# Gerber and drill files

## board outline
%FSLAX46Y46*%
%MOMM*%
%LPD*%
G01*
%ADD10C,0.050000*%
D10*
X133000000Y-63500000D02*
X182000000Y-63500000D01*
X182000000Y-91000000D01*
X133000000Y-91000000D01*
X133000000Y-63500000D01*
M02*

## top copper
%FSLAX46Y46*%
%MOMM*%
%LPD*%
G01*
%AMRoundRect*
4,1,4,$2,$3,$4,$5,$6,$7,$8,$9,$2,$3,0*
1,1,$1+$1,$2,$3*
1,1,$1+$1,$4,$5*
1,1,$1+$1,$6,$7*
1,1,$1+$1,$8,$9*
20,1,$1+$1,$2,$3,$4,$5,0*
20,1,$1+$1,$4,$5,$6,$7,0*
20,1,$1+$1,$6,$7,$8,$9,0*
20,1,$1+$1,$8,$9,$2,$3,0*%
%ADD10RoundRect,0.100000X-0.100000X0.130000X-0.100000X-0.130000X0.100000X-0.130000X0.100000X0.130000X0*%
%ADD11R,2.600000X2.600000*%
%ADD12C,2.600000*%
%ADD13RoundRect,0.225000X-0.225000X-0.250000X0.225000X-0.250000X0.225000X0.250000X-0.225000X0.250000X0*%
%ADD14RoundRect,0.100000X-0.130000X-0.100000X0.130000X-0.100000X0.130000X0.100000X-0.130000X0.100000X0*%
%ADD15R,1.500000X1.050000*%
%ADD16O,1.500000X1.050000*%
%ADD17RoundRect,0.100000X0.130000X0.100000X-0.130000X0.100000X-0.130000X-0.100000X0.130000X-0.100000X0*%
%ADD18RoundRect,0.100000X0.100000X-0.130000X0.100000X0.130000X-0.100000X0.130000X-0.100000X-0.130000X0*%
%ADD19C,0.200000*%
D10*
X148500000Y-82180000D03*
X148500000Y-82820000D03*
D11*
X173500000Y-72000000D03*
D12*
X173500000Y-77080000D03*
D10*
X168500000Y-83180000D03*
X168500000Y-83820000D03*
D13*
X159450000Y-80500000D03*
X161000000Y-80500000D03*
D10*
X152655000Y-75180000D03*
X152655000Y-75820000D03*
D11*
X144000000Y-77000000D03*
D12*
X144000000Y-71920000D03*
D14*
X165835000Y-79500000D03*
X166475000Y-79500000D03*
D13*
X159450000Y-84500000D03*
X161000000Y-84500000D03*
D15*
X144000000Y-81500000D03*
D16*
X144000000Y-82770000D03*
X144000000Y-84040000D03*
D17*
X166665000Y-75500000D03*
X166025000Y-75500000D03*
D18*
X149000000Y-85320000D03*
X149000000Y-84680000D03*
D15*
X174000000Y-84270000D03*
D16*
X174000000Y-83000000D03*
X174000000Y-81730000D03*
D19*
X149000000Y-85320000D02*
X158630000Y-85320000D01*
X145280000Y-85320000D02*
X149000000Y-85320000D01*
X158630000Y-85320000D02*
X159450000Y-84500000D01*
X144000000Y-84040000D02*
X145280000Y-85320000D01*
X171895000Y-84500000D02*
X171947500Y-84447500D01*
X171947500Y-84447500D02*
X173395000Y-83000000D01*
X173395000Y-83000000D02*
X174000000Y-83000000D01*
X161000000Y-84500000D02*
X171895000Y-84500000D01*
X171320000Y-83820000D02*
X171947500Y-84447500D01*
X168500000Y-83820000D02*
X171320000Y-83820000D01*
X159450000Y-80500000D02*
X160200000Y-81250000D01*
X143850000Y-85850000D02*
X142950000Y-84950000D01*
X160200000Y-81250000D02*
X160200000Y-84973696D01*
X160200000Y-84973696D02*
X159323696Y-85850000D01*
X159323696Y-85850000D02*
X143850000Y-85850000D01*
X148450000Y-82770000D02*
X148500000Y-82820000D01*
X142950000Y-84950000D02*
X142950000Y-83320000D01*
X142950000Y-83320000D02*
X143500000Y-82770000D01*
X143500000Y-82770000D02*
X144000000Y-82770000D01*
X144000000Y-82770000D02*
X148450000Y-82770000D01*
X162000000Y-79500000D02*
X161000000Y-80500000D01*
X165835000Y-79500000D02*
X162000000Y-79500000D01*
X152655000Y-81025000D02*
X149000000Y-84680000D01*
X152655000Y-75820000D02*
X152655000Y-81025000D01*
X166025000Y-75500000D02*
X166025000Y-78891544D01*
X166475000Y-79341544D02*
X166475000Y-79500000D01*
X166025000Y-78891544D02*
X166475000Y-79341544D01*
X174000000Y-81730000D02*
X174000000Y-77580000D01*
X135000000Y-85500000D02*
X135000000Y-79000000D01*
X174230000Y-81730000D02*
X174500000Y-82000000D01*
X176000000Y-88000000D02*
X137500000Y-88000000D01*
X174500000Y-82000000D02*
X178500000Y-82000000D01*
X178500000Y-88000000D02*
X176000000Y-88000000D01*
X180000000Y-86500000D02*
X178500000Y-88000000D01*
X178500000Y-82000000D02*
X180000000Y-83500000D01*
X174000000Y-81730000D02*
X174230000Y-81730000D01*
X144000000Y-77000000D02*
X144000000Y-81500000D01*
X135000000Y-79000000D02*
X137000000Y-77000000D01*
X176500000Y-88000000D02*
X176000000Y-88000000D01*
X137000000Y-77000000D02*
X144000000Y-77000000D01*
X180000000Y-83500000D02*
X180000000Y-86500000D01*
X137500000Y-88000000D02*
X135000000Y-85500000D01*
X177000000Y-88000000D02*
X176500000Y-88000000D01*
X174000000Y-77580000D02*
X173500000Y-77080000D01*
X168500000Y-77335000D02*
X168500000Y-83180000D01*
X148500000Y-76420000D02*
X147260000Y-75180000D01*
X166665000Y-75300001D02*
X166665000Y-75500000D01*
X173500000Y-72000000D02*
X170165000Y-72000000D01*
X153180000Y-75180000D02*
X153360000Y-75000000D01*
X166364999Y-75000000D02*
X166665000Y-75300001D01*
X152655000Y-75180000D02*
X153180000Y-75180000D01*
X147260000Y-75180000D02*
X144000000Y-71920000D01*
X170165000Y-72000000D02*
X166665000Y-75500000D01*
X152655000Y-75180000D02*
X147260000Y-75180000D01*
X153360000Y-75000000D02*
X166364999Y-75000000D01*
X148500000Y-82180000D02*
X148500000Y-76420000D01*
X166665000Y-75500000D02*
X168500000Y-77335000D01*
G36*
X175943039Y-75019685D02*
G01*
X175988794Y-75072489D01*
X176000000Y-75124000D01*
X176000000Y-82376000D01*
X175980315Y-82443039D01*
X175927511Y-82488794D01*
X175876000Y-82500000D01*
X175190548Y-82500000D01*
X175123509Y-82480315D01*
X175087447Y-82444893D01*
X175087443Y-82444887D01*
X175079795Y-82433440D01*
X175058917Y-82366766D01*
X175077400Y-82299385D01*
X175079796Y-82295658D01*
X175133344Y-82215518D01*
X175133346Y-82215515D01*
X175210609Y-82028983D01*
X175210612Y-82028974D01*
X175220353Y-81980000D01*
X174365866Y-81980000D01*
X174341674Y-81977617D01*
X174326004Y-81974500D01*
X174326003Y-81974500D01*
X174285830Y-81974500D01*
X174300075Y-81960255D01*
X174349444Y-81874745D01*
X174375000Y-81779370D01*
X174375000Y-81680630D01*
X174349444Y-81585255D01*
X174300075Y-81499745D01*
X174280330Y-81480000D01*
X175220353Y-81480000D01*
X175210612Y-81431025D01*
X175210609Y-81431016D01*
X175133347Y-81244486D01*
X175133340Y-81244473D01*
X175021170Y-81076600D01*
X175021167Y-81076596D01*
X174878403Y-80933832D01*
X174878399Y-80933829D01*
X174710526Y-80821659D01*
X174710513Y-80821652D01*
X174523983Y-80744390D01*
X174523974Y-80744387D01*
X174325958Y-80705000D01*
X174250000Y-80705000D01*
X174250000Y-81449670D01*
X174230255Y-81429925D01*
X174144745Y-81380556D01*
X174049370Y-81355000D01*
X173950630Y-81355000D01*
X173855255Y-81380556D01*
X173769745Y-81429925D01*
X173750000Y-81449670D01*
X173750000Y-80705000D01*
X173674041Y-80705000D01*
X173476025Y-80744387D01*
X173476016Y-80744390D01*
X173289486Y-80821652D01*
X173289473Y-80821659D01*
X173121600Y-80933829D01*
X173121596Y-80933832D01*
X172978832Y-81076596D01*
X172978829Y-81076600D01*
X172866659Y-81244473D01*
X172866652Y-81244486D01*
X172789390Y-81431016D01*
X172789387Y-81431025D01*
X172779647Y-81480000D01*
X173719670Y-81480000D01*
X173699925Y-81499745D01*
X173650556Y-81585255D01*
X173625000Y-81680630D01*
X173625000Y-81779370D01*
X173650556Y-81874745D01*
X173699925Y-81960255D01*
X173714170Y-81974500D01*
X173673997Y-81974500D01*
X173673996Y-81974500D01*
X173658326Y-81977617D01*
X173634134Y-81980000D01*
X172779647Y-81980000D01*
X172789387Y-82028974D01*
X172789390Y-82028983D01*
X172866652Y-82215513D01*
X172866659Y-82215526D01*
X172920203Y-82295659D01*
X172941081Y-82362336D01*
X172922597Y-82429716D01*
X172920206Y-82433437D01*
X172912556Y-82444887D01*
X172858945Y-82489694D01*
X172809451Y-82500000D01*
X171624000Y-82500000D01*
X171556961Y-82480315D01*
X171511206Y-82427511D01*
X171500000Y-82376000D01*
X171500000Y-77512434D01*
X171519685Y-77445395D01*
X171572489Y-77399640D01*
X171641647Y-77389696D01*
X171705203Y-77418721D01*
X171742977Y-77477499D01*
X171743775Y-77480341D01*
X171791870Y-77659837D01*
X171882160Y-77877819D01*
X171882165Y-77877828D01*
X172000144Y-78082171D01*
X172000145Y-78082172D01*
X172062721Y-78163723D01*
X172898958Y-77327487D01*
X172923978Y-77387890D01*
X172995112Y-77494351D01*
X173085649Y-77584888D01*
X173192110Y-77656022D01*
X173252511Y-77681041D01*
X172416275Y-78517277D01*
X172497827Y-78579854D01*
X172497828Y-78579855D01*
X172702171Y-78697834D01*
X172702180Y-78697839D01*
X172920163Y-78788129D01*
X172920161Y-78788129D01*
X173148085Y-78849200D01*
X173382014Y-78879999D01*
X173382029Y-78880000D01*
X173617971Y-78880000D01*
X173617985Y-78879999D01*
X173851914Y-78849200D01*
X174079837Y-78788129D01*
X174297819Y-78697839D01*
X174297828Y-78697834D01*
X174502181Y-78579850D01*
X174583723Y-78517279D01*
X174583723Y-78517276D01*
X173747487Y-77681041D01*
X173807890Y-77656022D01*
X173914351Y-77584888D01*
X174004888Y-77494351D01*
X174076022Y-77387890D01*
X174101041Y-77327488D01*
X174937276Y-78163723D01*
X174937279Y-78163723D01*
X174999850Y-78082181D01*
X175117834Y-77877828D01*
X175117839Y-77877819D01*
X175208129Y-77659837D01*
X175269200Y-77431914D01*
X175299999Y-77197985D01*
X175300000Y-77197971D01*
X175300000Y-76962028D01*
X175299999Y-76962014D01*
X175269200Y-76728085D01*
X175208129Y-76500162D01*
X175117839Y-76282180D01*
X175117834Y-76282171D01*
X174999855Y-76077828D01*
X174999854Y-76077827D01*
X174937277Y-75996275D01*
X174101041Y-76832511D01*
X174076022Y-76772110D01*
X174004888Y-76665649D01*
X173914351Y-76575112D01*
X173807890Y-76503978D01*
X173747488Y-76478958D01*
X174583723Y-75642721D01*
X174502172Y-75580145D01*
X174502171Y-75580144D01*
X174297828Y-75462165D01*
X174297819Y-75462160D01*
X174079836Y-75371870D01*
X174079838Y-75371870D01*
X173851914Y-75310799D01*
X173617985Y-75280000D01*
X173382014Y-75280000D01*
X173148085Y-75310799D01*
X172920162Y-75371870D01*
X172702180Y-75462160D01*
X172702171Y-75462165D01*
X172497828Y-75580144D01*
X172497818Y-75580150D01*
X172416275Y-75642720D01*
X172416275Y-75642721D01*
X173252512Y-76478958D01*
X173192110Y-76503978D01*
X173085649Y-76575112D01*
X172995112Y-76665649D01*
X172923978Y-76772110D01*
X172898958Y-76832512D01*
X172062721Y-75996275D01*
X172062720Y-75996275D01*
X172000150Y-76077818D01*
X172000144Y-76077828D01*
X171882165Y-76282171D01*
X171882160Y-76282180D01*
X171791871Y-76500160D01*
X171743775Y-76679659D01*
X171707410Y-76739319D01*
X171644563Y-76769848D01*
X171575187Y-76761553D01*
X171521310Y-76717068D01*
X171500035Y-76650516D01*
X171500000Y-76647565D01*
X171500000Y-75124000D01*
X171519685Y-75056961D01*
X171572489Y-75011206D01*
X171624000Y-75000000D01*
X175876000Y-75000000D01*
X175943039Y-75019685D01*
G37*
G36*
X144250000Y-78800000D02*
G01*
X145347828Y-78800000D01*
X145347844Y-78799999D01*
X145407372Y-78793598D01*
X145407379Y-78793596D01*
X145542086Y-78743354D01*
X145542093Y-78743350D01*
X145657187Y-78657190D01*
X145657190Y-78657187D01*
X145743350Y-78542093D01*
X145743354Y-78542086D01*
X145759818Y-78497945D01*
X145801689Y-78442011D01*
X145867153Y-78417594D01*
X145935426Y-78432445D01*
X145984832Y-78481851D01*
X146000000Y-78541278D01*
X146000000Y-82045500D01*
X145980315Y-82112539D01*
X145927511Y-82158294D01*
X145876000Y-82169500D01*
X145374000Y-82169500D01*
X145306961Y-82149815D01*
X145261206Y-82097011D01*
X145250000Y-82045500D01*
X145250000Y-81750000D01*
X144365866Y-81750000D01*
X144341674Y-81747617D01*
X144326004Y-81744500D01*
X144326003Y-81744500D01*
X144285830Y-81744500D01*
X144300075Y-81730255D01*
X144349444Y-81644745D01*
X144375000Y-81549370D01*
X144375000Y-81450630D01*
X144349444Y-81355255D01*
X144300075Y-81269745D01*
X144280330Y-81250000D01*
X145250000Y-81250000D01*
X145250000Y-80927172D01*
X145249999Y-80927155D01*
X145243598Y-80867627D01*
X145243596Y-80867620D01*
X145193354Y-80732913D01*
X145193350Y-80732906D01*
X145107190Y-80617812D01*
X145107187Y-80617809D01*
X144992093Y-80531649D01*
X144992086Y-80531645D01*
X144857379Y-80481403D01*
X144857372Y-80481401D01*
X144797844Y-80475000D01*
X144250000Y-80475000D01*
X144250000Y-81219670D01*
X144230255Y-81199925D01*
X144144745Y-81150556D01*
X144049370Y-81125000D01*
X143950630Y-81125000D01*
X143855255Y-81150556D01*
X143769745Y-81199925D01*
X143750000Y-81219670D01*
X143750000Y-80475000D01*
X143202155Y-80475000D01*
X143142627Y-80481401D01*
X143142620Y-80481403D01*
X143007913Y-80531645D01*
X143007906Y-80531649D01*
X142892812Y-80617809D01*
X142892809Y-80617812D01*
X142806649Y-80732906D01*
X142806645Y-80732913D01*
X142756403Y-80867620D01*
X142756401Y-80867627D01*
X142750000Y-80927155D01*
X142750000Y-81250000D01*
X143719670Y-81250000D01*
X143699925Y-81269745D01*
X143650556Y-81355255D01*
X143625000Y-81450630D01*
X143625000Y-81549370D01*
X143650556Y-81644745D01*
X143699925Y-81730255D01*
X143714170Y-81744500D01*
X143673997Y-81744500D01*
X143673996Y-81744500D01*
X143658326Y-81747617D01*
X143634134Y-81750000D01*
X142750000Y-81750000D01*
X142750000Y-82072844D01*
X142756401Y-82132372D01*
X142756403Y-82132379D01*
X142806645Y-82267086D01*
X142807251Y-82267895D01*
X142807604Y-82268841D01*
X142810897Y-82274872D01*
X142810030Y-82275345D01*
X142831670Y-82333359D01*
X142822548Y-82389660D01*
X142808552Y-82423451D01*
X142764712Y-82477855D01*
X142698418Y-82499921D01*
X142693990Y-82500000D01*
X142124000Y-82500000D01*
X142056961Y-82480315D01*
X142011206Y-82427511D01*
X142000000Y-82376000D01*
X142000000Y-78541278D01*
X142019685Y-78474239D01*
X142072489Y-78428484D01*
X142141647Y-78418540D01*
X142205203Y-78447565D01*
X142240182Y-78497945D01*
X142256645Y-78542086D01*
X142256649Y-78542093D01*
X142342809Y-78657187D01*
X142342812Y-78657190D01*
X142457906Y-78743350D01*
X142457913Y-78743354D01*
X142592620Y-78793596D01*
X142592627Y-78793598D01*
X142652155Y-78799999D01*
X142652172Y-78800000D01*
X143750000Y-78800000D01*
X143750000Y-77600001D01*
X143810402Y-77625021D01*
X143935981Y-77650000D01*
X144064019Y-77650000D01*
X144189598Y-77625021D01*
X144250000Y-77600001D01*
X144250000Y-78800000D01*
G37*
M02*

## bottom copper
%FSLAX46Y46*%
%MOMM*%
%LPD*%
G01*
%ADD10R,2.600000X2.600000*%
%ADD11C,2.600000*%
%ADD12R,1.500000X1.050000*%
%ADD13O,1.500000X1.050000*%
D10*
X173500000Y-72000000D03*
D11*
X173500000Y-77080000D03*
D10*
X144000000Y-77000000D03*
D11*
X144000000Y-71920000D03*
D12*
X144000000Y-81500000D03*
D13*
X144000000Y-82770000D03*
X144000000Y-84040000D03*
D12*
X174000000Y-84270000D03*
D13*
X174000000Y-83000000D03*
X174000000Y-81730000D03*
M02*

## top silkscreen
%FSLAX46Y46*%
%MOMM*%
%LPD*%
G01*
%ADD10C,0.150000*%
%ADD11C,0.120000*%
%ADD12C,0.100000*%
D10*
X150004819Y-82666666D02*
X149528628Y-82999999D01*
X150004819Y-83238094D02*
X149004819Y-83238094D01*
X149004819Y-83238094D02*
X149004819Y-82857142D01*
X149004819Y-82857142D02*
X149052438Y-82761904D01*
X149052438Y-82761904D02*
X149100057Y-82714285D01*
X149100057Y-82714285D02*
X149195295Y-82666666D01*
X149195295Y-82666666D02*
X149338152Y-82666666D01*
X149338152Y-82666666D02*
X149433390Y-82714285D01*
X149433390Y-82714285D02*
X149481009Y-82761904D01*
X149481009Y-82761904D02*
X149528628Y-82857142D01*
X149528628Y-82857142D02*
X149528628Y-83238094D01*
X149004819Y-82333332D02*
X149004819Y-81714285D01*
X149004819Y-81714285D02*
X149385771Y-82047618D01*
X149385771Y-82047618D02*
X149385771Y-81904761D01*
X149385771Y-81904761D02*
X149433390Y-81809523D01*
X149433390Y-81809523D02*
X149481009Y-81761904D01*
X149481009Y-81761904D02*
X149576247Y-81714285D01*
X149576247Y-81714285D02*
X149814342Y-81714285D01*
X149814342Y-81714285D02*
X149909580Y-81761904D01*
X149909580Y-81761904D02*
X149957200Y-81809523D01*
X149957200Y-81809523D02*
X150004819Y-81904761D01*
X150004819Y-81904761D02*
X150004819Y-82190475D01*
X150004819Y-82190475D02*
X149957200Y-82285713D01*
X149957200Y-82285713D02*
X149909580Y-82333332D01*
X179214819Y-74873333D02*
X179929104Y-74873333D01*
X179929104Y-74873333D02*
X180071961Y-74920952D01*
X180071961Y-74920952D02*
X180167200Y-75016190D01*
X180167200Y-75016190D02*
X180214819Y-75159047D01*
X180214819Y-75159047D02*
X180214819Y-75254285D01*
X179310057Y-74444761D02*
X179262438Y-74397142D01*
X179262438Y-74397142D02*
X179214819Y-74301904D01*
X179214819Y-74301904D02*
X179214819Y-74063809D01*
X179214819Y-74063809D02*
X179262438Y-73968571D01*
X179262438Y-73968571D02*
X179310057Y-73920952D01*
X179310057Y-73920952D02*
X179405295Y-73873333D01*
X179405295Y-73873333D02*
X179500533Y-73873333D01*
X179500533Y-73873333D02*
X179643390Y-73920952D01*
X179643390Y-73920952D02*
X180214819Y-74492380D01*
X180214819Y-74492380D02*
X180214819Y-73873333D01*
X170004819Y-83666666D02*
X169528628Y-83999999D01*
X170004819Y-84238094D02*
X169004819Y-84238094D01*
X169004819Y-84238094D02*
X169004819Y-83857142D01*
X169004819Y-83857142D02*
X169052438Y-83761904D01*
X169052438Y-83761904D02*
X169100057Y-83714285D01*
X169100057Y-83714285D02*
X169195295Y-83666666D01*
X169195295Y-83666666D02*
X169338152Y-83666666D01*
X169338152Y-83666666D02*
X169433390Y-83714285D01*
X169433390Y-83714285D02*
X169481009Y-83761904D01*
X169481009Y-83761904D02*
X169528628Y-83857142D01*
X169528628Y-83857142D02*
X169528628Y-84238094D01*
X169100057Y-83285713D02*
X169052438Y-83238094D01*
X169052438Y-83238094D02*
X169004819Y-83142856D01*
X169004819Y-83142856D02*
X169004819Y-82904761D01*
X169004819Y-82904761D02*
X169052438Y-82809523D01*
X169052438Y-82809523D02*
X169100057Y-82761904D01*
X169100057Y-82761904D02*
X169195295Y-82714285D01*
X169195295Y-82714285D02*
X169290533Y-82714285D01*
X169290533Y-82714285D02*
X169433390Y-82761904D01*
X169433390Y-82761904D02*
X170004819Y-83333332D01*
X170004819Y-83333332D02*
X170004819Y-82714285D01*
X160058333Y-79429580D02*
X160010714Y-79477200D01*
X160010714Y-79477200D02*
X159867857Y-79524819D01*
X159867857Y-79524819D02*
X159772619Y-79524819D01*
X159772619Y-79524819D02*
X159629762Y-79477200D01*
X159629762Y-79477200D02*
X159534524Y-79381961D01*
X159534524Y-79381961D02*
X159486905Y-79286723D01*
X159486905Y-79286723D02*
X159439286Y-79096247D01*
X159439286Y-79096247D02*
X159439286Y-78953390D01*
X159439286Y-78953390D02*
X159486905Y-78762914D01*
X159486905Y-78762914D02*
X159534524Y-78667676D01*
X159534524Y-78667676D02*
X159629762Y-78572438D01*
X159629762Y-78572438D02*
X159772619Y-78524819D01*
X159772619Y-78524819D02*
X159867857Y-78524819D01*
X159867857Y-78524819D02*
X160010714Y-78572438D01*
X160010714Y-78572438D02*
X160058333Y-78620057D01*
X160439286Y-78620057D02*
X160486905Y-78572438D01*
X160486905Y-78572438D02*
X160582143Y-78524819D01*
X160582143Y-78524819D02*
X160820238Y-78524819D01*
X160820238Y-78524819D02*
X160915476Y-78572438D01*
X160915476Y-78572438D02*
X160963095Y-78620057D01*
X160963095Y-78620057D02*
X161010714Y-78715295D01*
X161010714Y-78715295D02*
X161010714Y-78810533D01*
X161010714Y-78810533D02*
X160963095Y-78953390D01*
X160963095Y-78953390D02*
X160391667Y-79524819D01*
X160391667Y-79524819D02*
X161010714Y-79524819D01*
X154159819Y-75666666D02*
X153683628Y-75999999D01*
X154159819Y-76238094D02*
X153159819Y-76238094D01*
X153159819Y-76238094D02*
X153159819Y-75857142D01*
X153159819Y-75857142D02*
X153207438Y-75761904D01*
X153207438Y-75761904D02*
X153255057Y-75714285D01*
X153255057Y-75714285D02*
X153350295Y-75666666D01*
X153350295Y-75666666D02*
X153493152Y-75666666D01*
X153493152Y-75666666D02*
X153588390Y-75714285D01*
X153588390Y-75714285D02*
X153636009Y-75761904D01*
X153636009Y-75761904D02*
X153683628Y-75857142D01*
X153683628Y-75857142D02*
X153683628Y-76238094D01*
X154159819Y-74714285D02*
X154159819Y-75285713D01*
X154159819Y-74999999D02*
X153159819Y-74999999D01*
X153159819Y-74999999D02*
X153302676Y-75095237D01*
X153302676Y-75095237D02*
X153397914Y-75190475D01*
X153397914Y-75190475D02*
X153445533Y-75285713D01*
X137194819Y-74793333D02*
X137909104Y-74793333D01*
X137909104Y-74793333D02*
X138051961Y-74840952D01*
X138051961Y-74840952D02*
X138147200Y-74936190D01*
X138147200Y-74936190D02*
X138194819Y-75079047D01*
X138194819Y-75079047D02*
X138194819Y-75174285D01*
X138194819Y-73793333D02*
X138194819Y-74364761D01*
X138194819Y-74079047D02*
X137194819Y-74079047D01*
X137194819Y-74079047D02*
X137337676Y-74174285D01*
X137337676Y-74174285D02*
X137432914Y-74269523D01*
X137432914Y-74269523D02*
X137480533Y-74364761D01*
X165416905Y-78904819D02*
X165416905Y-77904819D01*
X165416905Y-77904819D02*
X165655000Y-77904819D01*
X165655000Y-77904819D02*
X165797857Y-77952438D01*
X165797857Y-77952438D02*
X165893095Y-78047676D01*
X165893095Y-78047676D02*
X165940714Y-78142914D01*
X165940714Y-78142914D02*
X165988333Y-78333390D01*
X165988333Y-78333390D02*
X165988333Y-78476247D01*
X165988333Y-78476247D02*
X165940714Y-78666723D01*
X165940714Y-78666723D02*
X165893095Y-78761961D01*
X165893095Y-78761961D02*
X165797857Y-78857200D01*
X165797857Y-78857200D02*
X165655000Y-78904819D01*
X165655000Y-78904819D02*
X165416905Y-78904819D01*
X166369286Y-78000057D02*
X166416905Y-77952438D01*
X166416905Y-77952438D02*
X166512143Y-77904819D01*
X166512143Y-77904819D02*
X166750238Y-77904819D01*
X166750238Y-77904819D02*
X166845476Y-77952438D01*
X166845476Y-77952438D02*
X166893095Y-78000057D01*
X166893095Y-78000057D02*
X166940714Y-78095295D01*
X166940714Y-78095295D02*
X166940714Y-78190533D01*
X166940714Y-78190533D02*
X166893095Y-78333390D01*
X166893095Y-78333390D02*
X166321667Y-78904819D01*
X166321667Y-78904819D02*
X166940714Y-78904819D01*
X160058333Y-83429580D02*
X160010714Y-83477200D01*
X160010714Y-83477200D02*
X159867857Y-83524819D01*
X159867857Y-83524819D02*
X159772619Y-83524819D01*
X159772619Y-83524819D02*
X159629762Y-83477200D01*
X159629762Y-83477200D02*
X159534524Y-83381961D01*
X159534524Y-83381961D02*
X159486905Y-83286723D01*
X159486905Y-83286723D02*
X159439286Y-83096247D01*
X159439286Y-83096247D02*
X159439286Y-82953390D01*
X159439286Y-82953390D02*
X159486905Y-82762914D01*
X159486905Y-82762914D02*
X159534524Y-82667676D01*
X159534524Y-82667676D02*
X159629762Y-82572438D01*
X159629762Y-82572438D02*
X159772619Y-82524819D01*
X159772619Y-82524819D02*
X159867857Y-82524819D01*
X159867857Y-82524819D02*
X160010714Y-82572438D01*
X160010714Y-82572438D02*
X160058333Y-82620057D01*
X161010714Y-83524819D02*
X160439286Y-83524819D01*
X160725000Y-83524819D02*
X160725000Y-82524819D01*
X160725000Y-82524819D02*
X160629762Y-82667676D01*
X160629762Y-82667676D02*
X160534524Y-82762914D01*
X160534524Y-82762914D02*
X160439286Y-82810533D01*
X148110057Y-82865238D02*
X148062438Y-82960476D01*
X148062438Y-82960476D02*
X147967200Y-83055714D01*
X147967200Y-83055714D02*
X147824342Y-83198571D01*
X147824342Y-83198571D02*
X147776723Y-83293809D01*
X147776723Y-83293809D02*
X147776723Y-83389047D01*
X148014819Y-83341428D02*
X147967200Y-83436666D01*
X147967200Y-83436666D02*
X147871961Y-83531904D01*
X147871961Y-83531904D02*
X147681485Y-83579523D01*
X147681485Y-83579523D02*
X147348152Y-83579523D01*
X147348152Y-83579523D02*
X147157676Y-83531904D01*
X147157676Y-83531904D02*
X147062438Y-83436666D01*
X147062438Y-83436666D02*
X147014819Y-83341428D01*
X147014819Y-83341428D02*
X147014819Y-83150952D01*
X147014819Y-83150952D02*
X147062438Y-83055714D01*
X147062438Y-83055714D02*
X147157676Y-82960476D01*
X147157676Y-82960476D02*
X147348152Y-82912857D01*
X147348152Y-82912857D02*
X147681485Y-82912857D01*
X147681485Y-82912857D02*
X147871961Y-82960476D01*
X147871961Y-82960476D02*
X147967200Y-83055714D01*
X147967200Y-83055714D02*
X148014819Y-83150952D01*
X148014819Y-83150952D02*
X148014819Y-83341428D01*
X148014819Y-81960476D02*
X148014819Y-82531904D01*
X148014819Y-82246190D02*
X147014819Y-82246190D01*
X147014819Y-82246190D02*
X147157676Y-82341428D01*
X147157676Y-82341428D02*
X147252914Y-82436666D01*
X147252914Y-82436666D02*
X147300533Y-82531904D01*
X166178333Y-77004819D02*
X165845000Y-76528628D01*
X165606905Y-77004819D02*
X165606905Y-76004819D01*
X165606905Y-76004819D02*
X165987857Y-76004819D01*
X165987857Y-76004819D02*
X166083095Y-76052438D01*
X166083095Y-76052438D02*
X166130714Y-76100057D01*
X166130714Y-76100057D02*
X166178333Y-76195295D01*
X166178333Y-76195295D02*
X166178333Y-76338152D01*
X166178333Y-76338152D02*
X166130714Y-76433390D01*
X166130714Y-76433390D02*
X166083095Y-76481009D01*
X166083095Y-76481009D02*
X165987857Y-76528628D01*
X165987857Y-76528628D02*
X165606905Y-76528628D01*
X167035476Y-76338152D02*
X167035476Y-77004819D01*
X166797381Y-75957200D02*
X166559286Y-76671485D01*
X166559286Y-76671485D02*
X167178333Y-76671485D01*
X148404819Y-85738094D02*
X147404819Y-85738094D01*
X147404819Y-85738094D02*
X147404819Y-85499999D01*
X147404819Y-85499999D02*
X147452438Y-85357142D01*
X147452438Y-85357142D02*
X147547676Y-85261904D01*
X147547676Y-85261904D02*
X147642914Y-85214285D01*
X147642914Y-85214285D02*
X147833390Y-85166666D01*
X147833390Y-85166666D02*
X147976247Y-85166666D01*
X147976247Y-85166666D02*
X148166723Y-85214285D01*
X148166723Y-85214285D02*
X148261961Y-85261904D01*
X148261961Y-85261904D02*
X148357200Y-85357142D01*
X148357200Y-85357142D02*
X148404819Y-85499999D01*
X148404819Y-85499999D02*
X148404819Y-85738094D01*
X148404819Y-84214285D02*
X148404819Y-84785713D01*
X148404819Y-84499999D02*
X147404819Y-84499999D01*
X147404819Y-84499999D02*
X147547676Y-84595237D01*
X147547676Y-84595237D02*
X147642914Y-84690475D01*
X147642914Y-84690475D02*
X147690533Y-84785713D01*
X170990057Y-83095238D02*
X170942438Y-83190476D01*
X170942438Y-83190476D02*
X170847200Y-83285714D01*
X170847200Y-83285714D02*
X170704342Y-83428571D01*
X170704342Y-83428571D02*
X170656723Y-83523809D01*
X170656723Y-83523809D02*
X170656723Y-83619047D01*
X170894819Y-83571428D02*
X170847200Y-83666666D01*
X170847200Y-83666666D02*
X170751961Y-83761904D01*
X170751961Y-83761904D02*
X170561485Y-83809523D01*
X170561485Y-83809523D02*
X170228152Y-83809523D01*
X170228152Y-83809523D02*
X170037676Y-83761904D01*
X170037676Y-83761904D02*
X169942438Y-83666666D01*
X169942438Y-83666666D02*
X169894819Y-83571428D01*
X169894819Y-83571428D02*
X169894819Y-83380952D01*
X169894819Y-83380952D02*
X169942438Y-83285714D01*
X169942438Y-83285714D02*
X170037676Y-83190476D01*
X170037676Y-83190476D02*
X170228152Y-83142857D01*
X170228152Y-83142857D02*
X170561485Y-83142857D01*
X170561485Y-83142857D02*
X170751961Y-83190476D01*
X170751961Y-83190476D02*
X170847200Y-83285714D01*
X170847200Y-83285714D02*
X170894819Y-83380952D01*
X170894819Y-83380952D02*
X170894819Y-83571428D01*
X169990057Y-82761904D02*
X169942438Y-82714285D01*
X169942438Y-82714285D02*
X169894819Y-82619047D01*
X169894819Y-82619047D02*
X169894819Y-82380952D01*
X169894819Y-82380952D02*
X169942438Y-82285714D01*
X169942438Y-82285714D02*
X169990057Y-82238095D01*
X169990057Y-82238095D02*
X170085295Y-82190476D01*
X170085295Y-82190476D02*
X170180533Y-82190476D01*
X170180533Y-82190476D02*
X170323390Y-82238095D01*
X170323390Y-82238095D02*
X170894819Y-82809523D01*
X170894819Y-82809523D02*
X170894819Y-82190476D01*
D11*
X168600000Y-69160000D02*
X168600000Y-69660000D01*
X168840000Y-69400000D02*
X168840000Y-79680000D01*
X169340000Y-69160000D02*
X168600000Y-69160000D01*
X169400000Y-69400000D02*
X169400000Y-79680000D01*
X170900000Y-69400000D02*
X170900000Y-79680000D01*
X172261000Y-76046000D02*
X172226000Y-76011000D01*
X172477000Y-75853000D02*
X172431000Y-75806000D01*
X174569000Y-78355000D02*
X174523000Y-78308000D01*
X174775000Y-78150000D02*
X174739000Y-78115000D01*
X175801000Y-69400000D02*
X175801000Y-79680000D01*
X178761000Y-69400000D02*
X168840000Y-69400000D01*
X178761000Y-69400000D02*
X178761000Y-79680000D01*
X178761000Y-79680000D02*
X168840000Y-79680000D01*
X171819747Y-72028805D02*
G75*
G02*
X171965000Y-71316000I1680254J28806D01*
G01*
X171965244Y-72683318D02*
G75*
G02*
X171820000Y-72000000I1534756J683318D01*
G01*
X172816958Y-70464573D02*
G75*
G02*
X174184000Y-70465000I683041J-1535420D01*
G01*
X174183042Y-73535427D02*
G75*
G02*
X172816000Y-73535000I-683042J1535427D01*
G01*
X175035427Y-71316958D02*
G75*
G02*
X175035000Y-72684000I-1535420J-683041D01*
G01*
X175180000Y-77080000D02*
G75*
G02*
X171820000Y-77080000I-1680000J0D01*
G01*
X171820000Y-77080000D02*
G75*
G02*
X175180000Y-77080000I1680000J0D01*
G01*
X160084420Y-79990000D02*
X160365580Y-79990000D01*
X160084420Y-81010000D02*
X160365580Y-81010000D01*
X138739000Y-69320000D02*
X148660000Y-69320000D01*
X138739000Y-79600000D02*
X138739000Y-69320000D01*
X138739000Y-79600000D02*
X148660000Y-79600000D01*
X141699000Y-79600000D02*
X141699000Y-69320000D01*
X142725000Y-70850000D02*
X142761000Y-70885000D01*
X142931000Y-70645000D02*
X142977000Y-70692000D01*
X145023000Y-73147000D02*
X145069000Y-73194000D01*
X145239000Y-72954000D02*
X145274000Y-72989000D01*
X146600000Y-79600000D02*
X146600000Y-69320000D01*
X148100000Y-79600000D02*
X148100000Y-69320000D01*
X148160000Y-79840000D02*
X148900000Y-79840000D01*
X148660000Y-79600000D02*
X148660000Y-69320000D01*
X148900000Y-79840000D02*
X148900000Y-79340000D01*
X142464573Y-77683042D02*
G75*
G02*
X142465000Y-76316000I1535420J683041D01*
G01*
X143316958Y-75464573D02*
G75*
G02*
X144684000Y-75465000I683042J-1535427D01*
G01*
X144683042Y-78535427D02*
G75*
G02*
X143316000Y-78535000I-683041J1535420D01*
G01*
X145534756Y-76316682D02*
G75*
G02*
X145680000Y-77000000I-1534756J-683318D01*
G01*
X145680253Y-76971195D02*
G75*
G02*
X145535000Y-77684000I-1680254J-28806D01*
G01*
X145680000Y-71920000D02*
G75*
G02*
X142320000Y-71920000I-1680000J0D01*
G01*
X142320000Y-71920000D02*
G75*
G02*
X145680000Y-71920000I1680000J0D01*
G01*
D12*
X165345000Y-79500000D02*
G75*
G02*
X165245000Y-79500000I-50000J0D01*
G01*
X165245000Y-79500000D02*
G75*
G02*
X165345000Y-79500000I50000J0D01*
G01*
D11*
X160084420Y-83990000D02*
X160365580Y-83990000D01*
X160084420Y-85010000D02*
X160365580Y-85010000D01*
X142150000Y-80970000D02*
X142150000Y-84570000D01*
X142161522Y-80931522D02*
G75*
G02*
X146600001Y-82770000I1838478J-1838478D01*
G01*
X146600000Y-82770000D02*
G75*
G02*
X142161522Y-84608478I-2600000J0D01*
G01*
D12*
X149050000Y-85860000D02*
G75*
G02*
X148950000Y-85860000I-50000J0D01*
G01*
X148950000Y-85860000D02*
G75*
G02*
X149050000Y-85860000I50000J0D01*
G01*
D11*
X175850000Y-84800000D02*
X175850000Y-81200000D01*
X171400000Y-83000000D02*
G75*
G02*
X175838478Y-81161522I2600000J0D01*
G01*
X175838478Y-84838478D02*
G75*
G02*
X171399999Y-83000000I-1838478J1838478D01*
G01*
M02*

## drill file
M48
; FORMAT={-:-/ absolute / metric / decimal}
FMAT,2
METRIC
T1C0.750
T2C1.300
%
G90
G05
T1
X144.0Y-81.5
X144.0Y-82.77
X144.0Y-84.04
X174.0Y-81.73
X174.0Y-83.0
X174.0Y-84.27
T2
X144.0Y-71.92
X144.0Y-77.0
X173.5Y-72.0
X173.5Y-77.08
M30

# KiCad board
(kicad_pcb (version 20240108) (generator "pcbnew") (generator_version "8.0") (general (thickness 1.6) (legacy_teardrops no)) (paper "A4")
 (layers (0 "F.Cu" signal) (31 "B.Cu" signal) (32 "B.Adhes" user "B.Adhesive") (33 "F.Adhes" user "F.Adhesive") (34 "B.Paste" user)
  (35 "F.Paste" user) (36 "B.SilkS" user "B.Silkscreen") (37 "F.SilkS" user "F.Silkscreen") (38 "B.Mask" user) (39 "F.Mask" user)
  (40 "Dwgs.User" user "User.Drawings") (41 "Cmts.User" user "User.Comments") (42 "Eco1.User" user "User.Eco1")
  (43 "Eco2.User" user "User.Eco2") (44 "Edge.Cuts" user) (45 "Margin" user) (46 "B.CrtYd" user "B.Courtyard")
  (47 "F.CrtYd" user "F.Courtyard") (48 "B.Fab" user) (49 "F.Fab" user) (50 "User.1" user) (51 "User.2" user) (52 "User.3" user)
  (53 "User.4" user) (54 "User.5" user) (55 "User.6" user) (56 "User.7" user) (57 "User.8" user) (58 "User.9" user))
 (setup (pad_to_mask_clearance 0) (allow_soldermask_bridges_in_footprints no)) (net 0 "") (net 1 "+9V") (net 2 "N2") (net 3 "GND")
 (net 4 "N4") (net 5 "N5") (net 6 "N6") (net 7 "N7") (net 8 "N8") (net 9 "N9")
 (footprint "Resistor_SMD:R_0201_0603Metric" (layer "F.Cu") (at 148.5 82.5 -90)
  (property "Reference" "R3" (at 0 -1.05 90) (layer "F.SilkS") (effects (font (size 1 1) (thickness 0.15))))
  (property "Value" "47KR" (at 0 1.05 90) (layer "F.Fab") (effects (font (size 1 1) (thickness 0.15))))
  (pad "" smd roundrect (at -0.345 0 270) (size 0.318 0.36) (layers "F.Paste") (roundrect_rratio 0.25))
  (pad "" smd roundrect (at 0.345 0 270) (size 0.318 0.36) (layers "F.Paste") (roundrect_rratio 0.25))
  (pad "1" smd roundrect (at -0.32 0 270) (size 0.46 0.4) (layers "F.Cu" "F.Mask") (roundrect_rratio 0.25) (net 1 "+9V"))
  (pad "2" smd roundrect (at 0.32 0 270) (size 0.46 0.4) (layers "F.Cu" "F.Mask") (roundrect_rratio 0.25) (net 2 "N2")))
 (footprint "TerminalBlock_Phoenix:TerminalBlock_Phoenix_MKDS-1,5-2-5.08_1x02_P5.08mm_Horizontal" (layer "F.Cu") (at 173.5 72 -90)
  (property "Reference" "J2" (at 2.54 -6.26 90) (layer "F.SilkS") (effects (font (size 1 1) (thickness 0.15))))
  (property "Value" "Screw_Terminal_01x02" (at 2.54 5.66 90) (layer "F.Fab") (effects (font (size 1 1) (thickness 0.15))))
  (fp_line (start -2.84 4.9) (end -2.34 4.9) (stroke (width 0.12) (type solid)) (layer "F.SilkS"))
  (fp_line (start -2.6 4.66) (end 7.68 4.66) (stroke (width 0.12) (type solid)) (layer "F.SilkS"))
  (fp_line (start -2.84 4.16) (end -2.84 4.9) (stroke (width 0.12) (type solid)) (layer "F.SilkS"))
  (fp_line (start -2.6 4.1) (end 7.68 4.1) (stroke (width 0.12) (type solid)) (layer "F.SilkS"))
  (fp_line (start -2.6 2.6) (end 7.68 2.6) (stroke (width 0.12) (type solid)) (layer "F.SilkS"))
  (fp_line (start 4.046 1.239) (end 4.011 1.274) (stroke (width 0.12) (type solid)) (layer "F.SilkS"))
  (fp_line (start 3.853 1.023) (end 3.806 1.069) (stroke (width 0.12) (type solid)) (layer "F.SilkS"))
  (fp_line (start 6.355 -1.069) (end 6.308 -1.023) (stroke (width 0.12) (type solid)) (layer "F.SilkS"))
  (fp_line (start 6.15 -1.275) (end 6.115 -1.239) (stroke (width 0.12) (type solid)) (layer "F.SilkS"))
  (fp_line (start -2.6 -2.301) (end 7.68 -2.301) (stroke (width 0.12) (type solid)) (layer "F.SilkS"))
  (fp_line (start -2.6 -5.261) (end -2.6 4.66) (stroke (width 0.12) (type solid)) (layer "F.SilkS"))
  (fp_line (start -2.6 -5.261) (end 7.68 -5.261) (stroke (width 0.12) (type solid)) (layer "F.SilkS"))
  (fp_line (start 7.68 -5.261) (end 7.68 4.66) (stroke (width 0.12) (type solid)) (layer "F.SilkS"))
  (fp_arc (start 0.028805 1.680253) (mid -0.335551 1.646659) (end -0.684 1.535) (stroke (width 0.12) (type solid)) (layer "F.SilkS"))
  (fp_arc (start 0.683318 1.534756) (mid 0.349292 1.643288) (end 0 1.68) (stroke (width 0.12) (type solid)) (layer "F.SilkS"))
  (fp_arc (start -1.535427 0.683042) (mid -1.680501 -0.000524) (end -1.535 -0.684) (stroke (width 0.12) (type solid)) (layer "F.SilkS"))
  (fp_arc (start 1.535427 -0.683042) (mid 1.680501 0.000524) (end 1.535 0.684) (stroke (width 0.12) (type solid)) (layer "F.SilkS"))
  (fp_arc (start -0.683042 -1.535427) (mid 0.000524 -1.680501) (end 0.684 -1.535) (stroke (width 0.12) (type solid)) (layer "F.SilkS"))
  (fp_circle (center 5.08 0) (end 6.76 0) (stroke (width 0.12) (type solid)) (fill none) (layer "F.SilkS"))
  (pad "1" thru_hole rect (at 0 0 270) (size 2.6 2.6) (drill 1.3) (layers "*.Cu" "*.Mask") (remove_unused_layers no) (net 1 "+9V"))
  (pad "2" thru_hole circle (at 5.08 0 270) (size 2.6 2.6) (drill 1.3) (layers "*.Cu" "*.Mask") (remove_unused_layers no) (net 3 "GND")))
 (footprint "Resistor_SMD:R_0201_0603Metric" (layer "F.Cu") (at 168.5 83.5 -90)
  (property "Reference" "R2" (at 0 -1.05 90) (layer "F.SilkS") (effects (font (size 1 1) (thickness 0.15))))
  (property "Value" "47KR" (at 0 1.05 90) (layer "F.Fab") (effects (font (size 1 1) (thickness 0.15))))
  (pad "" smd roundrect (at -0.345 0 270) (size 0.318 0.36) (layers "F.Paste") (roundrect_rratio 0.25))
  (pad "" smd roundrect (at 0.345 0 270) (size 0.318 0.36) (layers "F.Paste") (roundrect_rratio 0.25))
  (pad "1" smd roundrect (at -0.32 0 270) (size 0.46 0.4) (layers "F.Cu" "F.Mask") (roundrect_rratio 0.25) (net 1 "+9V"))
  (pad "2" smd roundrect (at 0.32 0 270) (size 0.46 0.4) (layers "F.Cu" "F.Mask") (roundrect_rratio 0.25) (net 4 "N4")))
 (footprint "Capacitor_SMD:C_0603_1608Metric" (layer "F.Cu") (at 160.225 80.5)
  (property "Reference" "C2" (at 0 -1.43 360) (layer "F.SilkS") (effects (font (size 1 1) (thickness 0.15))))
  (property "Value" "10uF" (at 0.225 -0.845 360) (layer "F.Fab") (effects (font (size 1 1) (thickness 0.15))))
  (fp_line (start -0.14058 -0.51) (end 0.14058 -0.51) (stroke (width 0.12) (type solid)) (layer "F.SilkS"))
  (fp_line (start -0.14058 0.51) (end 0.14058 0.51) (stroke (width 0.12) (type solid)) (layer "F.SilkS"))
  (pad "1" smd roundrect (at -0.775 0) (size 0.9 0.95) (layers "F.Cu" "F.Paste" "F.Mask") (roundrect_rratio 0.25) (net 2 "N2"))
  (pad "2" smd roundrect (at 0.775 0) (size 0.9 0.95) (layers "F.Cu" "F.Paste" "F.Mask") (roundrect_rratio 0.25) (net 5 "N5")))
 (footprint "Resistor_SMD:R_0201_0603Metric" (layer "F.Cu") (at 152.655 75.5 -90)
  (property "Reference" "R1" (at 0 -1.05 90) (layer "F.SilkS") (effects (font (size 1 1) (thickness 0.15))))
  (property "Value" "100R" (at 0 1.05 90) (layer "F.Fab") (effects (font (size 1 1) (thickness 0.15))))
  (pad "" smd roundrect (at -0.345 0 270) (size 0.318 0.36) (layers "F.Paste") (roundrect_rratio 0.25))
  (pad "" smd roundrect (at 0.345 0 270) (size 0.318 0.36) (layers "F.Paste") (roundrect_rratio 0.25))
  (pad "1" smd roundrect (at -0.32 0 270) (size 0.46 0.4) (layers "F.Cu" "F.Mask") (roundrect_rratio 0.25) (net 1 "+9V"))
  (pad "2" smd roundrect (at 0.32 0 270) (size 0.46 0.4) (layers "F.Cu" "F.Mask") (roundrect_rratio 0.25) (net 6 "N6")))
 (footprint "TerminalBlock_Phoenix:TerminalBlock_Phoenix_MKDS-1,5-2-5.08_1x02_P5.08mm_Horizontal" (layer "F.Cu") (at 144 77 90)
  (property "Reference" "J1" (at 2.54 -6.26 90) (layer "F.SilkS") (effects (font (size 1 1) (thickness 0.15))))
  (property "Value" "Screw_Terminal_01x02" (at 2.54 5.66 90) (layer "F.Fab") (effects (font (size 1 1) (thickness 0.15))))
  (fp_line (start 7.68 -5.261) (end 7.68 4.66) (stroke (width 0.12) (type solid)) (layer "F.SilkS"))
  (fp_line (start -2.6 -5.261) (end 7.68 -5.261) (stroke (width 0.12) (type solid)) (layer "F.SilkS"))
  (fp_line (start -2.6 -5.261) (end -2.6 4.66) (stroke (width 0.12) (type solid)) (layer "F.SilkS"))
  (fp_line (start -2.6 -2.301) (end 7.68 -2.301) (stroke (width 0.12) (type solid)) (layer "F.SilkS"))
  (fp_line (start 6.15 -1.275) (end 6.115 -1.239) (stroke (width 0.12) (type solid)) (layer "F.SilkS"))
  (fp_line (start 6.355 -1.069) (end 6.308 -1.023) (stroke (width 0.12) (type solid)) (layer "F.SilkS"))
  (fp_line (start 3.853 1.023) (end 3.806 1.069) (stroke (width 0.12) (type solid)) (layer "F.SilkS"))
  (fp_line (start 4.046 1.239) (end 4.011 1.274) (stroke (width 0.12) (type solid)) (layer "F.SilkS"))
  (fp_line (start -2.6 2.6) (end 7.68 2.6) (stroke (width 0.12) (type solid)) (layer "F.SilkS"))
  (fp_line (start -2.6 4.1) (end 7.68 4.1) (stroke (width 0.12) (type solid)) (layer "F.SilkS"))
  (fp_line (start -2.84 4.16) (end -2.84 4.9) (stroke (width 0.12) (type solid)) (layer "F.SilkS"))
  (fp_line (start -2.6 4.66) (end 7.68 4.66) (stroke (width 0.12) (type solid)) (layer "F.SilkS"))
  (fp_line (start -2.84 4.9) (end -2.34 4.9) (stroke (width 0.12) (type solid)) (layer "F.SilkS"))
  (fp_arc (start -0.683042 -1.535427) (mid 0.000524 -1.680501) (end 0.684 -1.535) (stroke (width 0.12) (type solid)) (layer "F.SilkS"))
  (fp_arc (start 1.535427 -0.683042) (mid 1.680501 0.000524) (end 1.535 0.684) (stroke (width 0.12) (type solid)) (layer "F.SilkS"))
  (fp_arc (start -1.535427 0.683042) (mid -1.680501 -0.000524) (end -1.535 -0.684) (stroke (width 0.12) (type solid)) (layer "F.SilkS"))
  (fp_arc (start 0.683318 1.534756) (mid 0.349292 1.643288) (end 0 1.68) (stroke (width 0.12) (type solid)) (layer "F.SilkS"))
  (fp_arc (start 0.028805 1.680253) (mid -0.335551 1.646659) (end -0.684 1.535) (stroke (width 0.12) (type solid)) (layer "F.SilkS"))
  (fp_circle (center 5.08 0) (end 6.76 0) (stroke (width 0.12) (type solid)) (fill none) (layer "F.SilkS"))
  (pad "1" thru_hole rect (at 0 0 90) (size 2.6 2.6) (drill 1.3) (layers "*.Cu" "*.Mask") (remove_unused_layers no) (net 3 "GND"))
  (pad "2" thru_hole circle (at 5.08 0 90) (size 2.6 2.6) (drill 1.3) (layers "*.Cu" "*.Mask") (remove_unused_layers no) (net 1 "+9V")))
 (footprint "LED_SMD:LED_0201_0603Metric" (layer "F.Cu") (at 166.155 79.5)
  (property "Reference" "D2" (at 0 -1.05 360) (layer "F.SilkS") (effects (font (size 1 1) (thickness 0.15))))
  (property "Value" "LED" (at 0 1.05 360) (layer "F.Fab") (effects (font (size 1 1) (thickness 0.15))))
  (fp_circle (center -0.86 0) (end -0.81 0) (stroke (width 0.1) (type solid)) (fill none) (layer "F.SilkS"))
  (pad "" smd roundrect (at -0.345 0) (size 0.318 0.36) (layers "F.Paste") (roundrect_rratio 0.25))
  (pad "" smd roundrect (at 0.345 0) (size 0.318 0.36) (layers "F.Paste") (roundrect_rratio 0.25))
  (pad "1" smd roundrect (at -0.32 0) (size 0.46 0.4) (layers "F.Cu" "F.Mask") (roundrect_rratio 0.25) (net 5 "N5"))
  (pad "2" smd roundrect (at 0.32 0) (size 0.46 0.4) (layers "F.Cu" "F.Mask") (roundrect_rratio 0.25) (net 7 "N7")))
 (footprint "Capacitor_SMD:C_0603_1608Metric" (layer "F.Cu") (at 160.225 84.5)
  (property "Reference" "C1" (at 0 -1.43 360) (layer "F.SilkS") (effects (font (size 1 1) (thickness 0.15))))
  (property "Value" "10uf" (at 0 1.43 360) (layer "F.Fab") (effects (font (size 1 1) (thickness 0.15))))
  (fp_line (start -0.14058 -0.51) (end 0.14058 -0.51) (stroke (width 0.12) (type solid)) (layer "F.SilkS"))
  (fp_line (start -0.14058 0.51) (end 0.14058 0.51) (stroke (width 0.12) (type solid)) (layer "F.SilkS"))
  (pad "1" smd roundrect (at -0.775 0) (size 0.9 0.95) (layers "F.Cu" "F.Paste" "F.Mask") (roundrect_rratio 0.25) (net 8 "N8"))
  (pad "2" smd roundrect (at 0.775 0) (size 0.9 0.95) (layers "F.Cu" "F.Paste" "F.Mask") (roundrect_rratio 0.25) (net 4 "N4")))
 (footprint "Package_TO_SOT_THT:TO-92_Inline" (layer "F.Cu") (at 144 81.5 -90)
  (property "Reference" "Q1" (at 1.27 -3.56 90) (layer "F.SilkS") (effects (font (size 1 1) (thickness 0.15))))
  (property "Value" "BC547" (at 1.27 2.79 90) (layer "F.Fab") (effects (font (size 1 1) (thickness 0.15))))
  (fp_line (start -0.53 1.85) (end 3.07 1.85) (stroke (width 0.12) (type solid)) (layer "F.SilkS"))
  (fp_arc (start -0.568478 1.838478) (mid -1.132087 -0.994977) (end 1.27 -2.6) (stroke (width 0.12) (type solid)) (layer "F.SilkS"))
  (fp_arc (start 1.27 -2.6) (mid 3.672087 -0.994977) (end 3.108478 1.838478) (stroke (width 0.12) (type solid)) (layer "F.SilkS"))
  (pad "1" thru_hole rect (at 0 0 270) (size 1.05 1.5) (drill 0.75) (layers "*.Cu" "*.Mask") (remove_unused_layers no) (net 3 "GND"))
  (pad "2" thru_hole oval (at 1.27 0 270) (size 1.05 1.5) (drill 0.75) (layers "*.Cu" "*.Mask") (remove_unused_layers no) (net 2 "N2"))
  (pad "3" thru_hole oval (at 2.54 0 270) (size 1.05 1.5) (drill 0.75) (layers "*.Cu" "*.Mask") (remove_unused_layers no) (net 8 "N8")))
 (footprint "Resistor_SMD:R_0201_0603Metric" (layer "F.Cu") (at 166.345 75.5 180)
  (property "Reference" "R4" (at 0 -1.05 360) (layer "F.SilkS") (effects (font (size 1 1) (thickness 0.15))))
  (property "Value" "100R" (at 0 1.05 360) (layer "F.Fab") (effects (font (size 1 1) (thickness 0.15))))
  (pad "" smd roundrect (at -0.345 0 180) (size 0.318 0.36) (layers "F.Paste") (roundrect_rratio 0.25))
  (pad "" smd roundrect (at 0.345 0 180) (size 0.318 0.36) (layers "F.Paste") (roundrect_rratio 0.25))
  (pad "1" smd roundrect (at -0.32 0 180) (size 0.46 0.4) (layers "F.Cu" "F.Mask") (roundrect_rratio 0.25) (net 1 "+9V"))
  (pad "2" smd roundrect (at 0.32 0 180) (size 0.46 0.4) (layers "F.Cu" "F.Mask") (roundrect_rratio 0.25) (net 7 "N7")))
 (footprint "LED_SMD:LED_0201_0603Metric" (layer "F.Cu") (at 149 85 90)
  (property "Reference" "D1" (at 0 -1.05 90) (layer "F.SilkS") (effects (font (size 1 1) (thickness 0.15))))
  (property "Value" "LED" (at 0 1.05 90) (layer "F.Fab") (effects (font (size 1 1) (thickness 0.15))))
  (fp_circle (center -0.86 0) (end -0.81 0) (stroke (width 0.1) (type solid)) (fill none) (layer "F.SilkS"))
  (pad "" smd roundrect (at -0.345 0 90) (size 0.318 0.36) (layers "F.Paste") (roundrect_rratio 0.25))
  (pad "" smd roundrect (at 0.345 0 90) (size 0.318 0.36) (layers "F.Paste") (roundrect_rratio 0.25))
  (pad "1" smd roundrect (at -0.32 0 90) (size 0.46 0.4) (layers "F.Cu" "F.Mask") (roundrect_rratio 0.25) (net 8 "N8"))
  (pad "2" smd roundrect (at 0.32 0 90) (size 0.46 0.4) (layers "F.Cu" "F.Mask") (roundrect_rratio 0.25) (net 6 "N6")))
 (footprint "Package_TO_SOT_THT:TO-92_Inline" (layer "F.Cu") (at 174 84.27 90)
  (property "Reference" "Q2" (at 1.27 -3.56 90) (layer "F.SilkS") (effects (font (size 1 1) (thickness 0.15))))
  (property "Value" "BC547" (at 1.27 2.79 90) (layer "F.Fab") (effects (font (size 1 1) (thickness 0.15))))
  (fp_line (start -0.53 1.85) (end 3.07 1.85) (stroke (width 0.12) (type solid)) (layer "F.SilkS"))
  (fp_arc (start 1.27 -2.6) (mid 3.672087 -0.994977) (end 3.108478 1.838478) (stroke (width 0.12) (type solid)) (layer "F.SilkS"))
  (fp_arc (start -0.568478 1.838478) (mid -1.132087 -0.994977) (end 1.27 -2.6) (stroke (width 0.12) (type solid)) (layer "F.SilkS"))
  (pad "1" thru_hole rect (at 0 0 90) (size 1.05 1.5) (drill 0.75) (layers "*.Cu" "*.Mask") (remove_unused_layers no) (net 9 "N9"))
  (pad "2" thru_hole oval (at 1.27 0 90) (size 1.05 1.5) (drill 0.75) (layers "*.Cu" "*.Mask") (remove_unused_layers no) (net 4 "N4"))
  (pad "3" thru_hole oval (at 2.54 0 90) (size 1.05 1.5) (drill 0.75) (layers "*.Cu" "*.Mask") (remove_unused_layers no) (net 3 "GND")))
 (gr_rect (start 133 63.5) (end 182 91) (stroke (width 0.05) (type default)) (fill none) (layer "Edge.Cuts"))
 (segment (start 149 85.32) (end 158.63 85.32) (width 0.2) (layer "F.Cu") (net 8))
 (segment (start 145.28 85.32) (end 149 85.32) (width 0.2) (layer "F.Cu") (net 8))
 (segment (start 158.63 85.32) (end 159.45 84.5) (width 0.2) (layer "F.Cu") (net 8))
 (segment (start 144 84.04) (end 145.28 85.32) (width 0.2) (layer "F.Cu") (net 8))
 (segment (start 171.895 84.5) (end 171.9475 84.4475) (width 0.2) (layer "F.Cu") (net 4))
 (segment (start 171.9475 84.4475) (end 173.395 83) (width 0.2) (layer "F.Cu") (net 4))
 (segment (start 173.395 83) (end 174 83) (width 0.2) (layer "F.Cu") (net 4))
 (segment (start 161 84.5) (end 171.895 84.5) (width 0.2) (layer "F.Cu") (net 4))
 (segment (start 171.32 83.82) (end 171.9475 84.4475) (width 0.2) (layer "F.Cu") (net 4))
 (segment (start 168.5 83.82) (end 171.32 83.82) (width 0.2) (layer "F.Cu") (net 4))
 (segment (start 159.45 80.5) (end 160.2 81.25) (width 0.2) (layer "F.Cu") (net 2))
 (segment (start 143.85 85.85) (end 142.95 84.95) (width 0.2) (layer "F.Cu") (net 2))
 (segment (start 160.2 81.25) (end 160.2 84.973696) (width 0.2) (layer "F.Cu") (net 2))
 (segment (start 160.2 84.973696) (end 159.323696 85.85) (width 0.2) (layer "F.Cu") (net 2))
 (segment (start 159.323696 85.85) (end 143.85 85.85) (width 0.2) (layer "F.Cu") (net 2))
 (segment (start 148.45 82.77) (end 148.5 82.82) (width 0.2) (layer "F.Cu") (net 2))
 (segment (start 142.95 84.95) (end 142.95 83.32) (width 0.2) (layer "F.Cu") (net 2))
 (segment (start 142.95 83.32) (end 143.5 82.77) (width 0.2) (layer "F.Cu") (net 2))
 (segment (start 143.5 82.77) (end 144 82.77) (width 0.2) (layer "F.Cu") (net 2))
 (segment (start 144 82.77) (end 148.45 82.77) (width 0.2) (layer "F.Cu") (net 2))
 (segment (start 162 79.5) (end 161 80.5) (width 0.2) (layer "F.Cu") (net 5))
 (segment (start 165.835 79.5) (end 162 79.5) (width 0.2) (layer "F.Cu") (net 5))
 (segment (start 152.655 81.025) (end 149 84.68) (width 0.2) (layer "F.Cu") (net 6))
 (segment (start 152.655 75.82) (end 152.655 81.025) (width 0.2) (layer "F.Cu") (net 6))
 (segment (start 166.025 75.5) (end 166.025 78.891544) (width 0.2) (layer "F.Cu") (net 7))
 (segment (start 166.475 79.341544) (end 166.475 79.5) (width 0.2) (layer "F.Cu") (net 7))
 (segment (start 166.025 78.891544) (end 166.475 79.341544) (width 0.2) (layer "F.Cu") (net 7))
 (segment (start 174 81.73) (end 174 77.58) (width 0.2) (layer "F.Cu") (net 3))
 (segment (start 135 85.5) (end 135 79) (width 0.2) (layer "F.Cu") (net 3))
 (segment (start 174.23 81.73) (end 174.5 82) (width 0.2) (layer "F.Cu") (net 3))
 (segment (start 176 88) (end 137.5 88) (width 0.2) (layer "F.Cu") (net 3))
 (segment (start 174.5 82) (end 178.5 82) (width 0.2) (layer "F.Cu") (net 3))
 (segment (start 178.5 88) (end 176 88) (width 0.2) (layer "F.Cu") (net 3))
 (segment (start 180 86.5) (end 178.5 88) (width 0.2) (layer "F.Cu") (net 3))
 (segment (start 178.5 82) (end 180 83.5) (width 0.2) (layer "F.Cu") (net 3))
 (segment (start 174 81.73) (end 174.23 81.73) (width 0.2) (layer "F.Cu") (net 3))
 (segment (start 144 77) (end 144 81.5) (width 0.2) (layer "F.Cu") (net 3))
 (segment (start 135 79) (end 137 77) (width 0.2) (layer "F.Cu") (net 3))
 (segment (start 176.5 88) (end 176 88) (width 0.2) (layer "F.Cu") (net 3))
 (segment (start 137 77) (end 144 77) (width 0.2) (layer "F.Cu") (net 3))
 (segment (start 180 83.5) (end 180 86.5) (width 0.2) (layer "F.Cu") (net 3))
 (segment (start 137.5 88) (end 135 85.5) (width 0.2) (layer "F.Cu") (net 3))
 (segment (start 177 88) (end 176.5 88) (width 0.2) (layer "F.Cu") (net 3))
 (segment (start 174 77.58) (end 173.5 77.08) (width 0.2) (layer "F.Cu") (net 3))
 (segment (start 168.5 77.335) (end 168.5 83.18) (width 0.2) (layer "F.Cu") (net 1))
 (segment (start 148.5 76.42) (end 147.26 75.18) (width 0.2) (layer "F.Cu") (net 1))
 (segment (start 166.665 75.300001) (end 166.665 75.5) (width 0.2) (layer "F.Cu") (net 1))
 (segment (start 173.5 72) (end 170.165 72) (width 0.2) (layer "F.Cu") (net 1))
 (segment (start 153.18 75.18) (end 153.36 75) (width 0.2) (layer "F.Cu") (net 1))
 (segment (start 166.364999 75) (end 166.665 75.300001) (width 0.2) (layer "F.Cu") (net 1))
 (segment (start 152.655 75.18) (end 153.18 75.18) (width 0.2) (layer "F.Cu") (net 1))
 (segment (start 147.26 75.18) (end 144 71.92) (width 0.2) (layer "F.Cu") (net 1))
 (segment (start 170.165 72) (end 166.665 75.5) (width 0.2) (layer "F.Cu") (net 1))
 (segment (start 152.655 75.18) (end 147.26 75.18) (width 0.2) (layer "F.Cu") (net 1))
 (segment (start 153.36 75) (end 166.364999 75) (width 0.2) (layer "F.Cu") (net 1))
 (segment (start 148.5 82.18) (end 148.5 76.42) (width 0.2) (layer "F.Cu") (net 1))
 (segment (start 166.665 75.5) (end 168.5 77.335) (width 0.2) (layer "F.Cu") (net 1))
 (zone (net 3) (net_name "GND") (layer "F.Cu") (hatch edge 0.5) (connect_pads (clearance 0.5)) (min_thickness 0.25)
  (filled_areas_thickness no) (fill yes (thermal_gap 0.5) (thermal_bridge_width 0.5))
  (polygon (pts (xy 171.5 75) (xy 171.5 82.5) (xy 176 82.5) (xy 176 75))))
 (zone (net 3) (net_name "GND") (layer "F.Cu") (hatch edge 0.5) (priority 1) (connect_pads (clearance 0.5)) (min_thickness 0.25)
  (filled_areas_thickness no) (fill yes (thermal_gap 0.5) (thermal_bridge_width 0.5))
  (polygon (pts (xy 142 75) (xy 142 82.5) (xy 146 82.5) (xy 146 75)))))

